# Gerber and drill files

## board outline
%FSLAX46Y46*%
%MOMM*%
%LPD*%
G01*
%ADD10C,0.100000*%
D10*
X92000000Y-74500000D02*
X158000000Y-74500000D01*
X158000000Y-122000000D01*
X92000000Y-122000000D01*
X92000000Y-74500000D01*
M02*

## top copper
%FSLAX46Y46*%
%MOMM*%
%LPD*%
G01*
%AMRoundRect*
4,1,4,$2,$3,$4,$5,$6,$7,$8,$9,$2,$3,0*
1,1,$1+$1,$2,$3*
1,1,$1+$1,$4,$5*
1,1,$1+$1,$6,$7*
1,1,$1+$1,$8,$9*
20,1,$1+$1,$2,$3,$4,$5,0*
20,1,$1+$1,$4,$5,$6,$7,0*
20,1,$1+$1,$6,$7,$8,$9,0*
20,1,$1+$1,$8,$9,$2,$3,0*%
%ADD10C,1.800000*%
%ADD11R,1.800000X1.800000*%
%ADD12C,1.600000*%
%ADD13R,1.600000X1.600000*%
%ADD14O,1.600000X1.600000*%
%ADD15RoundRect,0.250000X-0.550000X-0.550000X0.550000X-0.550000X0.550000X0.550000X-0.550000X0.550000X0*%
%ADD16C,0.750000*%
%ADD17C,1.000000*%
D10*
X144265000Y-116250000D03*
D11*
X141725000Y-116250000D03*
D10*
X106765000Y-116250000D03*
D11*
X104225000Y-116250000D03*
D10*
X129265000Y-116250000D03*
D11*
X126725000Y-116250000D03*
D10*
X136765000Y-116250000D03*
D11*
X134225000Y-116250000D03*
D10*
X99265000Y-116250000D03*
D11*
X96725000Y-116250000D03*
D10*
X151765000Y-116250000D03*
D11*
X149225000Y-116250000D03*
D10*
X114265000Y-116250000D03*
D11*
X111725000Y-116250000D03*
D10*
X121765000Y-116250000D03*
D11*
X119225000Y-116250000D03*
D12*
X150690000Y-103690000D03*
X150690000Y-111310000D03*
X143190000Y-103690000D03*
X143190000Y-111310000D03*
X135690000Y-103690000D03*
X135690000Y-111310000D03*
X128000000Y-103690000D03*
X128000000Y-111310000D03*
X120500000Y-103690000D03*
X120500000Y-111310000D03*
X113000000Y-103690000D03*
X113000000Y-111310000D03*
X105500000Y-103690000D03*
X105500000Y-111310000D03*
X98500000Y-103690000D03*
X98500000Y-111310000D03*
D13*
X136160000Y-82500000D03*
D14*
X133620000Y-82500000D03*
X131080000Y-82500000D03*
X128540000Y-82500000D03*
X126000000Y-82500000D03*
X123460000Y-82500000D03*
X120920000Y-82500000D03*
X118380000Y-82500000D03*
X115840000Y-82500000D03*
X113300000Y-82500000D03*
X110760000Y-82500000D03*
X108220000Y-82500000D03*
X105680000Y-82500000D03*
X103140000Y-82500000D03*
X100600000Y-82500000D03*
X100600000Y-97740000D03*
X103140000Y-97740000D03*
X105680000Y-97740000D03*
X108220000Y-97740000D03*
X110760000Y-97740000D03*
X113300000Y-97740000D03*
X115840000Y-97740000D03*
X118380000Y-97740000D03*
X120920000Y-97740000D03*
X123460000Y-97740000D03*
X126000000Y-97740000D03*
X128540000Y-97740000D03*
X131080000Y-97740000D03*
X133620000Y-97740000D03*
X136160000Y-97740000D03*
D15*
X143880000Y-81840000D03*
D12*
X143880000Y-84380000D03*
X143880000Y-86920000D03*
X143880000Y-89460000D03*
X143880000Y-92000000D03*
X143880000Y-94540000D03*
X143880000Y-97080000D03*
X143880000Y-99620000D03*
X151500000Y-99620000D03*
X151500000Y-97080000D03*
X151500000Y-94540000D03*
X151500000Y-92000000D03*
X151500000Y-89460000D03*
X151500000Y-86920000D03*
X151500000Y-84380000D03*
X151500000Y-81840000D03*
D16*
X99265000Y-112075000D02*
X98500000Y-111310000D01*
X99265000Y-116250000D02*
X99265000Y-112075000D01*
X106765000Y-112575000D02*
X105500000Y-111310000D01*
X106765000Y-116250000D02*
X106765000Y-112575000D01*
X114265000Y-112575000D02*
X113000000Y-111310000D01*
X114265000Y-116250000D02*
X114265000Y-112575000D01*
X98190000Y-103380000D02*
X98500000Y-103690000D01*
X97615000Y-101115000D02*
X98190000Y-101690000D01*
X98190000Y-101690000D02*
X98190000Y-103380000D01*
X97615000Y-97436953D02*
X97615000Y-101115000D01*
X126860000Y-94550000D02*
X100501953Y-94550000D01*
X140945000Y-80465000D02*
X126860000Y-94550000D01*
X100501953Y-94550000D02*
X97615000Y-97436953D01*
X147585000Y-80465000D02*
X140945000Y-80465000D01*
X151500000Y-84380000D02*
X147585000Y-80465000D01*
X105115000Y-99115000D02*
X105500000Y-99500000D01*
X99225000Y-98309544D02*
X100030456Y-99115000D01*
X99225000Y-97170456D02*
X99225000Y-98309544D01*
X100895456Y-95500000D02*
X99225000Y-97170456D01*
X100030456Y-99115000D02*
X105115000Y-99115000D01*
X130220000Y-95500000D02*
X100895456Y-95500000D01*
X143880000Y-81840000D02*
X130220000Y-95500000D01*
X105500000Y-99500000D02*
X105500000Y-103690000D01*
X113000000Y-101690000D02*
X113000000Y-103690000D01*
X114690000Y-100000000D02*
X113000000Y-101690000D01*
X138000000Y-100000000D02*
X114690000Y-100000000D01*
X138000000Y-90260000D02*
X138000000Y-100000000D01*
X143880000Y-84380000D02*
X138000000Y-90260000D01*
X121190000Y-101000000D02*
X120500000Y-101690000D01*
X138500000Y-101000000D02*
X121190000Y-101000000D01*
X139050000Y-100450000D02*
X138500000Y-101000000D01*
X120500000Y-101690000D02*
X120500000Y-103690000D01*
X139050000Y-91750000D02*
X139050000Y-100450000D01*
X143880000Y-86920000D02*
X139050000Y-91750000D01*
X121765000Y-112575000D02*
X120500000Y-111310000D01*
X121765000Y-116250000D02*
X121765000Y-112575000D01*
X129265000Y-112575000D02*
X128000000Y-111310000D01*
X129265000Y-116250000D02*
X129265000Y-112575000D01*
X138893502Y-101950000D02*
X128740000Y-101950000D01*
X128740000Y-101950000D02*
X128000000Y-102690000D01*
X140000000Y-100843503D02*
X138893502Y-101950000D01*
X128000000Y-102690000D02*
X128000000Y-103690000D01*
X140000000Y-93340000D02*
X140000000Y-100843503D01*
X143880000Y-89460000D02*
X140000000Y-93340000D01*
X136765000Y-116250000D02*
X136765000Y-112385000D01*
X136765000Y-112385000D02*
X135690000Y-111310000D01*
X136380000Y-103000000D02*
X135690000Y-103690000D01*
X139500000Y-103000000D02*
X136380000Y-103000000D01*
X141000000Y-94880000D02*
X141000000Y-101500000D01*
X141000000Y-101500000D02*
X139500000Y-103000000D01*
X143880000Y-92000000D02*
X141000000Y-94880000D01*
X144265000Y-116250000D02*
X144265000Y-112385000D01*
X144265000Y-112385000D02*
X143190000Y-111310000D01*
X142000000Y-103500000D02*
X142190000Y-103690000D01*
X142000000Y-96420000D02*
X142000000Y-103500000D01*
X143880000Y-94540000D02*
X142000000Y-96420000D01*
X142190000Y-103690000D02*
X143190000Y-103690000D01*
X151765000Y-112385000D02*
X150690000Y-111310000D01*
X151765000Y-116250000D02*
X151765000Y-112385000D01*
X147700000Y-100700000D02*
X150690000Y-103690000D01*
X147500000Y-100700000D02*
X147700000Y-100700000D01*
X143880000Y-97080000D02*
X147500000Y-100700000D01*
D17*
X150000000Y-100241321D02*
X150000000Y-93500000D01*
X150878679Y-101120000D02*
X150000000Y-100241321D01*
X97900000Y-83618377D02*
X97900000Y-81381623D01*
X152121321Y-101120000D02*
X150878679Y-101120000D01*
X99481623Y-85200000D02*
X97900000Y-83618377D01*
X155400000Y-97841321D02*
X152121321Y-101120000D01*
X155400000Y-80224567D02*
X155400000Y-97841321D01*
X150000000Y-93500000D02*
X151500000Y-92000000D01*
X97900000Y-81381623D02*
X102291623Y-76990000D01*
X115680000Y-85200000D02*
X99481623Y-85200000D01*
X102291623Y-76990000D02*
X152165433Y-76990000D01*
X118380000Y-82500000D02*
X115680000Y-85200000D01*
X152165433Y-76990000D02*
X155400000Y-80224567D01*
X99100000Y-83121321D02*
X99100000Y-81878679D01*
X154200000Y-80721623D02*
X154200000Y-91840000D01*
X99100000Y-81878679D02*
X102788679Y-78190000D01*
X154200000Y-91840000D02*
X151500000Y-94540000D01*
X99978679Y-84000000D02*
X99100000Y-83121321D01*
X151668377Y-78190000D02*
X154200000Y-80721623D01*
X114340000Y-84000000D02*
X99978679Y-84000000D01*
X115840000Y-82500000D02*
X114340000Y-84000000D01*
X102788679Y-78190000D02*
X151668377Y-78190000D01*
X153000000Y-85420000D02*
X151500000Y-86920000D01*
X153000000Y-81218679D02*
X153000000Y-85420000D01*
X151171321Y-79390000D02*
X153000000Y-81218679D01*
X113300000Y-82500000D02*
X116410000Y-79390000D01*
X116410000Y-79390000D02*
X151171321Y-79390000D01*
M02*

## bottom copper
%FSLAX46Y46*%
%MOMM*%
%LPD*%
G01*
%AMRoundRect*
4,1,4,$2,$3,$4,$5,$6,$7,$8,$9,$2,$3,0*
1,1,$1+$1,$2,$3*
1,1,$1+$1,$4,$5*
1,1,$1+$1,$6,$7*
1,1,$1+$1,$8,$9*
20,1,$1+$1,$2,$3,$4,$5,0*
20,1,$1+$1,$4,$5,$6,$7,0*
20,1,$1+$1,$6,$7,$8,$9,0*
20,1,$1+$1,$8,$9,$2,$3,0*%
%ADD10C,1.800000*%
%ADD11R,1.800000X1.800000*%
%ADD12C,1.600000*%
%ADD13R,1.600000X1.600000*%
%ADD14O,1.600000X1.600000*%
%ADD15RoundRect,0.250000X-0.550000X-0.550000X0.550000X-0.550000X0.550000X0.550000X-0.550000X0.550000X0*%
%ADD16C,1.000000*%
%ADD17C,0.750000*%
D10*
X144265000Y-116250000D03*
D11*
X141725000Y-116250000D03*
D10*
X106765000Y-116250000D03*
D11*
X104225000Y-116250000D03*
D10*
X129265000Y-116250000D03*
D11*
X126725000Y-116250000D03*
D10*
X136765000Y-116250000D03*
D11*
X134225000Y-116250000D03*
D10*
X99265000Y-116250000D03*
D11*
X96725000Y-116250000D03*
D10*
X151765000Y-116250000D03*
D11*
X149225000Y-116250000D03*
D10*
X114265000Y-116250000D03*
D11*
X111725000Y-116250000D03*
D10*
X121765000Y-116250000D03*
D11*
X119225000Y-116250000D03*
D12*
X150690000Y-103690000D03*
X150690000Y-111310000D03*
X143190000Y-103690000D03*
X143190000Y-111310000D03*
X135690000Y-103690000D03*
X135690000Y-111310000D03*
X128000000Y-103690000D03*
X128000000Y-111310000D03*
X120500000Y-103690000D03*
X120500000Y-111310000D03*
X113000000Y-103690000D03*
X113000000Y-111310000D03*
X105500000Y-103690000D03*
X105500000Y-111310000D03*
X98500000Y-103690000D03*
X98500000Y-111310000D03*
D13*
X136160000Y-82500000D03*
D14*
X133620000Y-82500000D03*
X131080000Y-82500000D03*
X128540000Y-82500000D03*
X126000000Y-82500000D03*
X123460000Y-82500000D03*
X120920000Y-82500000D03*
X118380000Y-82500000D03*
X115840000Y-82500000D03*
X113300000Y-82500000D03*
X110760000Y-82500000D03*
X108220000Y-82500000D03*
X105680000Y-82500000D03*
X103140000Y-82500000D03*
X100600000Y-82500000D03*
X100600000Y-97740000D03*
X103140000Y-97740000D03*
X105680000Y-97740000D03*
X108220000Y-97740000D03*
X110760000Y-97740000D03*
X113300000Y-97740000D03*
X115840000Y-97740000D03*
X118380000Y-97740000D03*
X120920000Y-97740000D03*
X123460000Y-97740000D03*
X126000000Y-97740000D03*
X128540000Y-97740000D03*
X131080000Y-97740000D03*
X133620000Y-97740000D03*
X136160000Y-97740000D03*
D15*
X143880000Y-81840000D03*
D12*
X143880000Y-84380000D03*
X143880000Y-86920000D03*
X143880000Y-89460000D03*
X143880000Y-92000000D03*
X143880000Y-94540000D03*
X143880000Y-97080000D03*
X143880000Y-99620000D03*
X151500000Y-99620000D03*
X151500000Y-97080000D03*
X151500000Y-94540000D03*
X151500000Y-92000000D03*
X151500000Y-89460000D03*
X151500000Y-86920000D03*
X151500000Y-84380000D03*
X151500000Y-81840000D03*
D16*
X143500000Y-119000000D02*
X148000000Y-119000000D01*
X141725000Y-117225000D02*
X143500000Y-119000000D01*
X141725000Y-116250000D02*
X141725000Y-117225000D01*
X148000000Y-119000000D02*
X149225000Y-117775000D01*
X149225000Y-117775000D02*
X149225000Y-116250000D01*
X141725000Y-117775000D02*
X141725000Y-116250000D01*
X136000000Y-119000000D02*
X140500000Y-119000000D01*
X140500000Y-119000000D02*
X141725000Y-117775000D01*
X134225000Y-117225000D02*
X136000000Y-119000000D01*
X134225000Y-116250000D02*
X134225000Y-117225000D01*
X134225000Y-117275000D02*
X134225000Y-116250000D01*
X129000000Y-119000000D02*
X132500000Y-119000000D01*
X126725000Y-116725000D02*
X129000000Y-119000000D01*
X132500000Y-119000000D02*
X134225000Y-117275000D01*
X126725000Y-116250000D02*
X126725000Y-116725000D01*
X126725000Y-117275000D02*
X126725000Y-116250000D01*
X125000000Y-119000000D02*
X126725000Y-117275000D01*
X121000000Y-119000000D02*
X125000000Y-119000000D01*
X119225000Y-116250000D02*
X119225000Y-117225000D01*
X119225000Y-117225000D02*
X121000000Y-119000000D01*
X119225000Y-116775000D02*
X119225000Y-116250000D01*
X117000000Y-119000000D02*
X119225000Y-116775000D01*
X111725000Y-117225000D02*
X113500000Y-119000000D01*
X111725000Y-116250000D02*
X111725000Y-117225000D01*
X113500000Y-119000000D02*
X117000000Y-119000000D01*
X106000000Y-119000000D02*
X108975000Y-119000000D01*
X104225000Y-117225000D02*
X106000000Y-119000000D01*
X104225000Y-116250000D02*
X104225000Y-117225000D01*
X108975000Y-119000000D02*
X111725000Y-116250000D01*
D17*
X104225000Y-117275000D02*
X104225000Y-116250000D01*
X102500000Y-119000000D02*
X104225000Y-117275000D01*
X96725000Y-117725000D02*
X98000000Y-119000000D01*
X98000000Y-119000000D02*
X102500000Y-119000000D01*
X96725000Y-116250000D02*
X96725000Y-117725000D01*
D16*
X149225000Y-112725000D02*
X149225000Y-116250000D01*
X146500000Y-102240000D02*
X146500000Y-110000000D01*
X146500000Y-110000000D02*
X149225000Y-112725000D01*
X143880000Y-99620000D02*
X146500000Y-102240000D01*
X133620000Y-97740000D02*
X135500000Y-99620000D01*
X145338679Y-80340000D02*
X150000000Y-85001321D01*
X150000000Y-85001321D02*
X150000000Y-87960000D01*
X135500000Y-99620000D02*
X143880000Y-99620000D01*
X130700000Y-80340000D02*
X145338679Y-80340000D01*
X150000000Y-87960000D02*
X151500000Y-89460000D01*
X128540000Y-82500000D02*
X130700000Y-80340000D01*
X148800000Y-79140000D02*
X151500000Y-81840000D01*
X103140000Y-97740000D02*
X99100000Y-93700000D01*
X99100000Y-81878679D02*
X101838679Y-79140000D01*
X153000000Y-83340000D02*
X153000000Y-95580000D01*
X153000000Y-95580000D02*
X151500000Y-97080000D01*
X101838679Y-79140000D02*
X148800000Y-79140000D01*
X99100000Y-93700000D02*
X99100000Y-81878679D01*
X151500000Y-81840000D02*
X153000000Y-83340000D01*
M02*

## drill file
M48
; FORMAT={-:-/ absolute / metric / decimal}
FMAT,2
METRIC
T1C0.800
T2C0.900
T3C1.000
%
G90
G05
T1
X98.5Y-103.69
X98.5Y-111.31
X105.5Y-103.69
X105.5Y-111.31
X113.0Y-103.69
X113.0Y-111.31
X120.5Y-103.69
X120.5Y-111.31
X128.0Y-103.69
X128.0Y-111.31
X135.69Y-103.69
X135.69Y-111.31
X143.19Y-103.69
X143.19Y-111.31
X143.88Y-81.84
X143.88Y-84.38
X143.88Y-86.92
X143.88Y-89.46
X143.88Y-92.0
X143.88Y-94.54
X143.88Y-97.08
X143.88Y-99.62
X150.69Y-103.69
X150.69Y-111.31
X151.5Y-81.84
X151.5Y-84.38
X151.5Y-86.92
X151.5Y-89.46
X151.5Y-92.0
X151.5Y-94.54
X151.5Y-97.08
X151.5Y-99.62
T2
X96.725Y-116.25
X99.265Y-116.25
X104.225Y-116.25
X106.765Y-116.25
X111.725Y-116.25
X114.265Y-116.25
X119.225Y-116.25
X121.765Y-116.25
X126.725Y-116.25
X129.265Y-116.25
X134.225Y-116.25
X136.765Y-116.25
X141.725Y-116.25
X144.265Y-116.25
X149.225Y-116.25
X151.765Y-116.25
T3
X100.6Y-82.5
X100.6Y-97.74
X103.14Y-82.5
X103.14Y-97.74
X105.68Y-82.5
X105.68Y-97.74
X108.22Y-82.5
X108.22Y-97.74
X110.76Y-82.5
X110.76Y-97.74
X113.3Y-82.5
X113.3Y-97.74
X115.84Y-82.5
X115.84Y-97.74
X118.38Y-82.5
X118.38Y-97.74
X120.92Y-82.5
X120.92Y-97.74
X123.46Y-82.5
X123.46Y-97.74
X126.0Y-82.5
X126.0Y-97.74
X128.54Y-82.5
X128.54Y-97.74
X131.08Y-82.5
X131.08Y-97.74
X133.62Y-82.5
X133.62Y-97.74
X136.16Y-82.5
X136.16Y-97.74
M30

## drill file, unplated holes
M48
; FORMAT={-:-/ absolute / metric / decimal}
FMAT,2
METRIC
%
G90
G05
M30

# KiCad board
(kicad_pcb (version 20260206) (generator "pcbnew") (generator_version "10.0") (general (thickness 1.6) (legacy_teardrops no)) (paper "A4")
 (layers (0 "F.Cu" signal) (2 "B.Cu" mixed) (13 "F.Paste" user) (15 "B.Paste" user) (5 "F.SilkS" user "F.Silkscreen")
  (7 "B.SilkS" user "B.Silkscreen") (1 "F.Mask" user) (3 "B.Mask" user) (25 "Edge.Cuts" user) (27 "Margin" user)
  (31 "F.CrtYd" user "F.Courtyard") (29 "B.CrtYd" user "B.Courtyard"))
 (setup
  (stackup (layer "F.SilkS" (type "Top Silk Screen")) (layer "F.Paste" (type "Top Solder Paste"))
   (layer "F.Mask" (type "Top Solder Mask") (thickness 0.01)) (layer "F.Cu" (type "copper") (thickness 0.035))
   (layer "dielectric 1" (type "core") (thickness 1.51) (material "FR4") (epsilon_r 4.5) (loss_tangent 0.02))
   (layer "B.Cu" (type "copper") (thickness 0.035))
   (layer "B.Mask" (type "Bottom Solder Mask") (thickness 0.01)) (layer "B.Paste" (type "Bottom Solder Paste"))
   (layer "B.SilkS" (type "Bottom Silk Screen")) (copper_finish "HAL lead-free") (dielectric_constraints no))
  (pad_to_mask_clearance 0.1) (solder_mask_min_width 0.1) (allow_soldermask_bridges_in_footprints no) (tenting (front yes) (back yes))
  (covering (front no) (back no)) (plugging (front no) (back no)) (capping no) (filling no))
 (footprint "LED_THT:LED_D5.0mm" (layer "F.Cu") (at 119.225 116.25)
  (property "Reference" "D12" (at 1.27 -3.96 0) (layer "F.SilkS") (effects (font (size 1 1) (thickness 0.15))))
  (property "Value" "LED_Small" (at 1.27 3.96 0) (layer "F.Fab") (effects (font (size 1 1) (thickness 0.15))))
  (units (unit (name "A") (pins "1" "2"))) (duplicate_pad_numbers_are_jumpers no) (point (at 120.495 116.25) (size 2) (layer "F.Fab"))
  (pad "1" thru_hole rect (at 0 0) (size 1.8 1.8) (drill 0.9) (layers "*.Cu" "*.Mask") (remove_unused_layers no) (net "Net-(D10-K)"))
  (pad "2" thru_hole circle (at 2.54 0) (size 1.8 1.8) (drill 0.9) (layers "*.Cu" "*.Mask") (remove_unused_layers no) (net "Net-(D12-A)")))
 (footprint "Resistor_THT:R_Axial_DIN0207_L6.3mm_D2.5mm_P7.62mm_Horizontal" (layer "F.Cu") (at 128 103.69 -90)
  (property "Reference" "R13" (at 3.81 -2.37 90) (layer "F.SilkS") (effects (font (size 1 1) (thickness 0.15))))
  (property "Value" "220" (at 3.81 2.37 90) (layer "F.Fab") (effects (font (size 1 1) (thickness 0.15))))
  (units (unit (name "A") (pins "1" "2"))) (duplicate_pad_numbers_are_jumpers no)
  (pad "1" thru_hole circle (at 0 0 270) (size 1.6 1.6) (drill 0.8) (layers "*.Cu" "*.Mask") (remove_unused_layers no) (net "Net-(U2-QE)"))
  (pad "2" thru_hole circle (at 7.62 0 270) (size 1.6 1.6) (drill 0.8) (layers "*.Cu" "*.Mask") (remove_unused_layers no)
   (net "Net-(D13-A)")))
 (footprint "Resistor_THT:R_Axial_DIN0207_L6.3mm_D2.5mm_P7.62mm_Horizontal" (layer "F.Cu") (at 150.69 103.69 -90)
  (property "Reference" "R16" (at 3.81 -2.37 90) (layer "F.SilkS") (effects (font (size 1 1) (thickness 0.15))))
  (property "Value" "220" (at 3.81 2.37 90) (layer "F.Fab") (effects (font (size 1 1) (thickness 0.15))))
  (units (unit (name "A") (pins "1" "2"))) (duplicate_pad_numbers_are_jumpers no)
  (pad "1" thru_hole circle (at 0 0 270) (size 1.6 1.6) (drill 0.8) (layers "*.Cu" "*.Mask") (remove_unused_layers no) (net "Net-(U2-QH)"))
  (pad "2" thru_hole circle (at 7.62 0 270) (size 1.6 1.6) (drill 0.8) (layers "*.Cu" "*.Mask") (remove_unused_layers no)
   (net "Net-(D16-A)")))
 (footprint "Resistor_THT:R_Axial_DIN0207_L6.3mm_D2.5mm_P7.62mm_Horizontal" (layer "F.Cu") (at 135.69 103.69 -90)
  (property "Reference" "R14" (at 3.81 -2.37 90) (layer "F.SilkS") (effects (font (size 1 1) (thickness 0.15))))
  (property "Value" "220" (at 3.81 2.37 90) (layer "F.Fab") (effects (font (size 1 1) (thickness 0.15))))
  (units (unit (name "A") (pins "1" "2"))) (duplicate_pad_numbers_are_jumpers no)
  (pad "1" thru_hole circle (at 0 0 270) (size 1.6 1.6) (drill 0.8) (layers "*.Cu" "*.Mask") (remove_unused_layers no) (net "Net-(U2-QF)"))
  (pad "2" thru_hole circle (at 7.62 0 270) (size 1.6 1.6) (drill 0.8) (layers "*.Cu" "*.Mask") (remove_unused_layers no)
   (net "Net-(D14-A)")))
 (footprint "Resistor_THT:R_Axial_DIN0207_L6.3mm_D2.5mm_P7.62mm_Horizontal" (layer "F.Cu") (at 113 103.69 -90)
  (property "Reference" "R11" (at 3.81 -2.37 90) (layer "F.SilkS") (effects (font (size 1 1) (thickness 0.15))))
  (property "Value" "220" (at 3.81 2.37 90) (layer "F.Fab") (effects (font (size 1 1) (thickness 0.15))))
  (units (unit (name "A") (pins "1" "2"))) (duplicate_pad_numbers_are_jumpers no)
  (pad "1" thru_hole circle (at 0 0 270) (size 1.6 1.6) (drill 0.8) (layers "*.Cu" "*.Mask") (remove_unused_layers no) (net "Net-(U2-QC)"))
  (pad "2" thru_hole circle (at 7.62 0 270) (size 1.6 1.6) (drill 0.8) (layers "*.Cu" "*.Mask") (remove_unused_layers no)
   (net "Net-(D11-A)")))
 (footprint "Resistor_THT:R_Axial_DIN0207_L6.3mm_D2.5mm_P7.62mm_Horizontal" (layer "F.Cu") (at 105.5 103.69 -90)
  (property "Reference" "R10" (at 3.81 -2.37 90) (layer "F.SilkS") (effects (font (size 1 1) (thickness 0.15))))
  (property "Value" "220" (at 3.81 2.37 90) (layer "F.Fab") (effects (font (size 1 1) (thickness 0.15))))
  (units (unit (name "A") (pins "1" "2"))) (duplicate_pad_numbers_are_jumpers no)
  (pad "1" thru_hole circle (at 0 0 270) (size 1.6 1.6) (drill 0.8) (layers "*.Cu" "*.Mask") (remove_unused_layers no) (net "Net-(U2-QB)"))
  (pad "2" thru_hole circle (at 7.62 0 270) (size 1.6 1.6) (drill 0.8) (layers "*.Cu" "*.Mask") (remove_unused_layers no)
   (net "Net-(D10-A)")))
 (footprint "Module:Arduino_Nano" (layer "F.Cu") (at 136.16 82.5 -90)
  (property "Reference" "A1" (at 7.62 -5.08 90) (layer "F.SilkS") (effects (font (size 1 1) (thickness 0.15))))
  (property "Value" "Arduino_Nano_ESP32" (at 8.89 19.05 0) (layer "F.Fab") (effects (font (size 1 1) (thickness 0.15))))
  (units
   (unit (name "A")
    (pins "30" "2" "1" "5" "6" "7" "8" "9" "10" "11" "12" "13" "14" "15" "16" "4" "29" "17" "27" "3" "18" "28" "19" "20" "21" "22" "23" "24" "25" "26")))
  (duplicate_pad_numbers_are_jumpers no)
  (pad "1" thru_hole rect (at 0 0 270) (size 1.6 1.6) (drill 1) (layers "*.Cu" "*.Mask") (remove_unused_layers no)
   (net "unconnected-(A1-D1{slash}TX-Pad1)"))
  (pad "2" thru_hole oval (at 0 2.54 270) (size 1.6 1.6) (drill 1) (layers "*.Cu" "*.Mask") (remove_unused_layers no)
   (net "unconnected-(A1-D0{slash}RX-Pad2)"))
  (pad "3" thru_hole oval (at 0 5.08 270) (size 1.6 1.6) (drill 1) (layers "*.Cu" "*.Mask") (remove_unused_layers no)
   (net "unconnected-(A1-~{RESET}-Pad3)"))
  (pad "4" thru_hole oval (at 0 7.62 270) (size 1.6 1.6) (drill 1) (layers "*.Cu" "*.Mask") (remove_unused_layers no) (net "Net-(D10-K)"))
  (pad "5" thru_hole oval (at 0 10.16 270) (size 1.6 1.6) (drill 1) (layers "*.Cu" "*.Mask") (remove_unused_layers no)
   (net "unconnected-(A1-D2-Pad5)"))
  (pad "6" thru_hole oval (at 0 12.7 270) (size 1.6 1.6) (drill 1) (layers "*.Cu" "*.Mask") (remove_unused_layers no)
   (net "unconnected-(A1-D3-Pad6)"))
  (pad "7" thru_hole oval (at 0 15.24 270) (size 1.6 1.6) (drill 1) (layers "*.Cu" "*.Mask") (remove_unused_layers no)
   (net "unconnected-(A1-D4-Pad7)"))
  (pad "8" thru_hole oval (at 0 17.78 270) (size 1.6 1.6) (drill 1) (layers "*.Cu" "*.Mask") (remove_unused_layers no) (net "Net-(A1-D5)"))
  (pad "9" thru_hole oval (at 0 20.32 270) (size 1.6 1.6) (drill 1) (layers "*.Cu" "*.Mask") (remove_unused_layers no) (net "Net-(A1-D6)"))
  (pad "10" thru_hole oval (at 0 22.86 270) (size 1.6 1.6) (drill 1) (layers "*.Cu" "*.Mask") (remove_unused_layers no) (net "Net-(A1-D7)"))
  (pad "11" thru_hole oval (at 0 25.4 270) (size 1.6 1.6) (drill 1) (layers "*.Cu" "*.Mask") (remove_unused_layers no)
   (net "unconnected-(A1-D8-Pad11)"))
  (pad "12" thru_hole oval (at 0 27.94 270) (size 1.6 1.6) (drill 1) (layers "*.Cu" "*.Mask") (remove_unused_layers no)
   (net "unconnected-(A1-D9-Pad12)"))
  (pad "13" thru_hole oval (at 0 30.48 270) (size 1.6 1.6) (drill 1) (layers "*.Cu" "*.Mask") (remove_unused_layers no)
   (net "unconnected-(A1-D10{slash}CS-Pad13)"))
  (pad "14" thru_hole oval (at 0 33.02 270) (size 1.6 1.6) (drill 1) (layers "*.Cu" "*.Mask") (remove_unused_layers no)
   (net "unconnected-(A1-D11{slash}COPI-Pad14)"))
  (pad "15" thru_hole oval (at 0 35.56 270) (size 1.6 1.6) (drill 1) (layers "*.Cu" "*.Mask") (remove_unused_layers no)
   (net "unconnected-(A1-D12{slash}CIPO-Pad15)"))
  (pad "16" thru_hole oval (at 15.24 35.56 270) (size 1.6 1.6) (drill 1) (layers "*.Cu" "*.Mask") (remove_unused_layers no)
   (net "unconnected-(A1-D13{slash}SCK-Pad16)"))
  (pad "17" thru_hole oval (at 15.24 33.02 270) (size 1.6 1.6) (drill 1) (layers "*.Cu" "*.Mask") (remove_unused_layers no)
   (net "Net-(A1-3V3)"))
  (pad "18" thru_hole oval (at 15.24 30.48 270) (size 1.6 1.6) (drill 1) (layers "*.Cu" "*.Mask") (remove_unused_layers no)
   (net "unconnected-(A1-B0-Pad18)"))
  (pad "19" thru_hole oval (at 15.24 27.94 270) (size 1.6 1.6) (drill 1) (layers "*.Cu" "*.Mask") (remove_unused_layers no)
   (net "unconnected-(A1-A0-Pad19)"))
  (pad "20" thru_hole oval (at 15.24 25.4 270) (size 1.6 1.6) (drill 1) (layers "*.Cu" "*.Mask") (remove_unused_layers no)
   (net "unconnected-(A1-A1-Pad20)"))
  (pad "21" thru_hole oval (at 15.24 22.86 270) (size 1.6 1.6) (drill 1) (layers "*.Cu" "*.Mask") (remove_unused_layers no)
   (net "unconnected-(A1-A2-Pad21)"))
  (pad "22" thru_hole oval (at 15.24 20.32 270) (size 1.6 1.6) (drill 1) (layers "*.Cu" "*.Mask") (remove_unused_layers no)
   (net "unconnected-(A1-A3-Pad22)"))
  (pad "23" thru_hole oval (at 15.24 17.78 270) (size 1.6 1.6) (drill 1) (layers "*.Cu" "*.Mask") (remove_unused_layers no)
   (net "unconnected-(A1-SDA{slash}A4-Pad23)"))
  (pad "24" thru_hole oval (at 15.24 15.24 270) (size 1.6 1.6) (drill 1) (layers "*.Cu" "*.Mask") (remove_unused_layers no)
   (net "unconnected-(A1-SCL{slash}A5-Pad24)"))
  (pad "25" thru_hole oval (at 15.24 12.7 270) (size 1.6 1.6) (drill 1) (layers "*.Cu" "*.Mask") (remove_unused_layers no)
   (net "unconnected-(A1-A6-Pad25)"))
  (pad "26" thru_hole oval (at 15.24 10.16 270) (size 1.6 1.6) (drill 1) (layers "*.Cu" "*.Mask") (remove_unused_layers no)
   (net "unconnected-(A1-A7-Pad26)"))
  (pad "27" thru_hole oval (at 15.24 7.62 270) (size 1.6 1.6) (drill 1) (layers "*.Cu" "*.Mask") (remove_unused_layers no)
   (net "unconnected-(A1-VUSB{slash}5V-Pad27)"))
  (pad "28" thru_hole oval (at 15.24 5.08 270) (size 1.6 1.6) (drill 1) (layers "*.Cu" "*.Mask") (remove_unused_layers no)
   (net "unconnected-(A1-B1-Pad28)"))
  (pad "29" thru_hole oval (at 15.24 2.54 270) (size 1.6 1.6) (drill 1) (layers "*.Cu" "*.Mask") (remove_unused_layers no)
   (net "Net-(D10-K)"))
  (pad "30" thru_hole oval (at 15.24 0 270) (size 1.6 1.6) (drill 1) (layers "*.Cu" "*.Mask") (remove_unused_layers no)
   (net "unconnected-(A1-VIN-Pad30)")))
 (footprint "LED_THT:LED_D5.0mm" (layer "F.Cu") (at 104.225 116.25)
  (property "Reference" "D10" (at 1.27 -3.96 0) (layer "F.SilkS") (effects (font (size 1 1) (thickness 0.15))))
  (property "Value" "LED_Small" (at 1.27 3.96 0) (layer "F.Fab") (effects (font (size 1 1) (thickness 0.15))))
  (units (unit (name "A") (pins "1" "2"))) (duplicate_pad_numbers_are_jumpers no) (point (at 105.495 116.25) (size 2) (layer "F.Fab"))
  (pad "1" thru_hole rect (at 0 0) (size 1.8 1.8) (drill 0.9) (layers "*.Cu" "*.Mask") (remove_unused_layers no) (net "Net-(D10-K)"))
  (pad "2" thru_hole circle (at 2.54 0) (size 1.8 1.8) (drill 0.9) (layers "*.Cu" "*.Mask") (remove_unused_layers no) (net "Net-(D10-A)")))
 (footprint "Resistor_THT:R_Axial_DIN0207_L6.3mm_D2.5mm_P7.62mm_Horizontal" (layer "F.Cu") (at 143.19 103.69 -90)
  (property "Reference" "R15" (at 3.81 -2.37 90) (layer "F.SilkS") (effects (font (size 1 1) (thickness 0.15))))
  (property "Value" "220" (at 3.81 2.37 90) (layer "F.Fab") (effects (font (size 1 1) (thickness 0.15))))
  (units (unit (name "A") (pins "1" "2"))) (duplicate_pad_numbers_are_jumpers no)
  (pad "1" thru_hole circle (at 0 0 270) (size 1.6 1.6) (drill 0.8) (layers "*.Cu" "*.Mask") (remove_unused_layers no) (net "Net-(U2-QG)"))
  (pad "2" thru_hole circle (at 7.62 0 270) (size 1.6 1.6) (drill 0.8) (layers "*.Cu" "*.Mask") (remove_unused_layers no)
   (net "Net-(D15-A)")))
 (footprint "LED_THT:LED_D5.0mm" (layer "F.Cu") (at 126.725 116.25)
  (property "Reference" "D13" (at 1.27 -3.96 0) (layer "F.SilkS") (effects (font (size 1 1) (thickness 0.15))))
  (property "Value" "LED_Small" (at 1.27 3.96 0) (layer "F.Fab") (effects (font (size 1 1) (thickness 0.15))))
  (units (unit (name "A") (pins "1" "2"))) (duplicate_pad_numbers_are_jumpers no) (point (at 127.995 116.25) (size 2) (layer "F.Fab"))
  (pad "1" thru_hole rect (at 0 0) (size 1.8 1.8) (drill 0.9) (layers "*.Cu" "*.Mask") (remove_unused_layers no) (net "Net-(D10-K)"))
  (pad "2" thru_hole circle (at 2.54 0) (size 1.8 1.8) (drill 0.9) (layers "*.Cu" "*.Mask") (remove_unused_layers no) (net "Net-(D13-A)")))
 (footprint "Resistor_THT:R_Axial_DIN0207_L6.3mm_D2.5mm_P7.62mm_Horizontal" (layer "F.Cu") (at 120.5 103.69 -90)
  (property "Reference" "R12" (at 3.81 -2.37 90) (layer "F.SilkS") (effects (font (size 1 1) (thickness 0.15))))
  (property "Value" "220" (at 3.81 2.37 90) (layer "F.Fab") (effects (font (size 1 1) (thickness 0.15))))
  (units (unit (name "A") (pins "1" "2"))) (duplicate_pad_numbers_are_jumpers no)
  (pad "1" thru_hole circle (at 0 0 270) (size 1.6 1.6) (drill 0.8) (layers "*.Cu" "*.Mask") (remove_unused_layers no) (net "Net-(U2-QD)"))
  (pad "2" thru_hole circle (at 7.62 0 270) (size 1.6 1.6) (drill 0.8) (layers "*.Cu" "*.Mask") (remove_unused_layers no)
   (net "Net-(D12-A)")))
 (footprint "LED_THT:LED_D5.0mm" (layer "F.Cu") (at 141.725 116.25)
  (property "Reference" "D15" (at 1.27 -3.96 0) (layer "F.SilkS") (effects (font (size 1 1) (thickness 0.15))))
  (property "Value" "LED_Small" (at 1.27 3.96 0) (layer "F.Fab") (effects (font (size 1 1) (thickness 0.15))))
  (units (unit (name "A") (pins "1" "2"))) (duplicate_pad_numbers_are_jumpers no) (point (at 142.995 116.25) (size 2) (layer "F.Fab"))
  (pad "1" thru_hole rect (at 0 0) (size 1.8 1.8) (drill 0.9) (layers "*.Cu" "*.Mask") (remove_unused_layers no) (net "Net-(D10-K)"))
  (pad "2" thru_hole circle (at 2.54 0) (size 1.8 1.8) (drill 0.9) (layers "*.Cu" "*.Mask") (remove_unused_layers no) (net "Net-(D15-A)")))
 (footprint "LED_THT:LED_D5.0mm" (layer "F.Cu") (at 111.725 116.25)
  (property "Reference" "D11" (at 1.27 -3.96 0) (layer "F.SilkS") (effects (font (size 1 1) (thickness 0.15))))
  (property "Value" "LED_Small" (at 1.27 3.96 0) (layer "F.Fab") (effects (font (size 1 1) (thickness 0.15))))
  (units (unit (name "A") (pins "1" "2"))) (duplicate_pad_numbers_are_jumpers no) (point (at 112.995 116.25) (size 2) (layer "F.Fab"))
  (pad "1" thru_hole rect (at 0 0) (size 1.8 1.8) (drill 0.9) (layers "*.Cu" "*.Mask") (remove_unused_layers no) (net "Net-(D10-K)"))
  (pad "2" thru_hole circle (at 2.54 0) (size 1.8 1.8) (drill 0.9) (layers "*.Cu" "*.Mask") (remove_unused_layers no) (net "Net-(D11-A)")))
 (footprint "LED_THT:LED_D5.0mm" (layer "F.Cu") (at 149.225 116.25)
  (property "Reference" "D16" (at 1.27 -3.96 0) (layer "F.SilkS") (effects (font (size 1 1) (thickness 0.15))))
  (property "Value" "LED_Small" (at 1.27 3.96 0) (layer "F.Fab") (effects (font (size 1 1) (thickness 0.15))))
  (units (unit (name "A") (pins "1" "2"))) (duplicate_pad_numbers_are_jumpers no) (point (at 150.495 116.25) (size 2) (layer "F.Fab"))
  (pad "1" thru_hole rect (at 0 0) (size 1.8 1.8) (drill 0.9) (layers "*.Cu" "*.Mask") (remove_unused_layers no) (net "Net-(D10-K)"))
  (pad "2" thru_hole circle (at 2.54 0) (size 1.8 1.8) (drill 0.9) (layers "*.Cu" "*.Mask") (remove_unused_layers no) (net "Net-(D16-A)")))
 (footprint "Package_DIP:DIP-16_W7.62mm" (layer "F.Cu") (at 143.88 81.84)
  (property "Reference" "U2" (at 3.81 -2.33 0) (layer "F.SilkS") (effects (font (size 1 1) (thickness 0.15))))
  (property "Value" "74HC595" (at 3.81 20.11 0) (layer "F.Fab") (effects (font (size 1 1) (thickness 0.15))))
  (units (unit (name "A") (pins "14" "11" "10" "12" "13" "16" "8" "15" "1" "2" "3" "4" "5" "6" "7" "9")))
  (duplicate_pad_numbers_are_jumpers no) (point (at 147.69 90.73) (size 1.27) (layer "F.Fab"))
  (pad "1" thru_hole roundrect (at 0 0) (size 1.6 1.6) (drill 0.8) (layers "*.Cu" "*.Mask") (remove_unused_layers no)
   (roundrect_rratio 0.15625) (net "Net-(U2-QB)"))
  (pad "2" thru_hole circle (at 0 2.54) (size 1.6 1.6) (drill 0.8) (layers "*.Cu" "*.Mask") (remove_unused_layers no) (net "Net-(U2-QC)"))
  (pad "3" thru_hole circle (at 0 5.08) (size 1.6 1.6) (drill 0.8) (layers "*.Cu" "*.Mask") (remove_unused_layers no) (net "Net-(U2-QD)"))
  (pad "4" thru_hole circle (at 0 7.62) (size 1.6 1.6) (drill 0.8) (layers "*.Cu" "*.Mask") (remove_unused_layers no) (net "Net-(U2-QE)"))
  (pad "5" thru_hole circle (at 0 10.16) (size 1.6 1.6) (drill 0.8) (layers "*.Cu" "*.Mask") (remove_unused_layers no) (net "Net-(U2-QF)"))
  (pad "6" thru_hole circle (at 0 12.7) (size 1.6 1.6) (drill 0.8) (layers "*.Cu" "*.Mask") (remove_unused_layers no) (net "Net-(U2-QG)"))
  (pad "7" thru_hole circle (at 0 15.24) (size 1.6 1.6) (drill 0.8) (layers "*.Cu" "*.Mask") (remove_unused_layers no) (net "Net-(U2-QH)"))
  (pad "8" thru_hole circle (at 0 17.78) (size 1.6 1.6) (drill 0.8) (layers "*.Cu" "*.Mask") (remove_unused_layers no) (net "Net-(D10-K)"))
  (pad "9" thru_hole circle (at 7.62 17.78) (size 1.6 1.6) (drill 0.8) (layers "*.Cu" "*.Mask") (remove_unused_layers no)
   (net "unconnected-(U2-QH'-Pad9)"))
  (pad "10" thru_hole circle (at 7.62 15.24) (size 1.6 1.6) (drill 0.8) (layers "*.Cu" "*.Mask") (remove_unused_layers no)
   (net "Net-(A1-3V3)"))
  (pad "11" thru_hole circle (at 7.62 12.7) (size 1.6 1.6) (drill 0.8) (layers "*.Cu" "*.Mask") (remove_unused_layers no)
   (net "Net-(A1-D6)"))
  (pad "12" thru_hole circle (at 7.62 10.16) (size 1.6 1.6) (drill 0.8) (layers "*.Cu" "*.Mask") (remove_unused_layers no)
   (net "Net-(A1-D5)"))
  (pad "13" thru_hole circle (at 7.62 7.62) (size 1.6 1.6) (drill 0.8) (layers "*.Cu" "*.Mask") (remove_unused_layers no)
   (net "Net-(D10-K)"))
  (pad "14" thru_hole circle (at 7.62 5.08) (size 1.6 1.6) (drill 0.8) (layers "*.Cu" "*.Mask") (remove_unused_layers no)
   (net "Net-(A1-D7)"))
  (pad "15" thru_hole circle (at 7.62 2.54) (size 1.6 1.6) (drill 0.8) (layers "*.Cu" "*.Mask") (remove_unused_layers no)
   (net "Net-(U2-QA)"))
  (pad "16" thru_hole circle (at 7.62 0) (size 1.6 1.6) (drill 0.8) (layers "*.Cu" "*.Mask") (remove_unused_layers no) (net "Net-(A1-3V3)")))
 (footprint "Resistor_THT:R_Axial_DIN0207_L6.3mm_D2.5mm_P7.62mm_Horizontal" (layer "F.Cu") (at 98.5 103.69 -90)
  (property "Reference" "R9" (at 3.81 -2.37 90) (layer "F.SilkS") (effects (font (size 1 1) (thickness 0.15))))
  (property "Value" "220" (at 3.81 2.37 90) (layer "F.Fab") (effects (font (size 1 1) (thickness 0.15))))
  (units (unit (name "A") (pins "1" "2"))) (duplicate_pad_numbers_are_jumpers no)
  (pad "1" thru_hole circle (at 0 0 270) (size 1.6 1.6) (drill 0.8) (layers "*.Cu" "*.Mask") (remove_unused_layers no) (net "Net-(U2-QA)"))
  (pad "2" thru_hole circle (at 7.62 0 270) (size 1.6 1.6) (drill 0.8) (layers "*.Cu" "*.Mask") (remove_unused_layers no) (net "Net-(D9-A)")))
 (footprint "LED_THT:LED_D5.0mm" (layer "F.Cu") (at 96.725 116.25)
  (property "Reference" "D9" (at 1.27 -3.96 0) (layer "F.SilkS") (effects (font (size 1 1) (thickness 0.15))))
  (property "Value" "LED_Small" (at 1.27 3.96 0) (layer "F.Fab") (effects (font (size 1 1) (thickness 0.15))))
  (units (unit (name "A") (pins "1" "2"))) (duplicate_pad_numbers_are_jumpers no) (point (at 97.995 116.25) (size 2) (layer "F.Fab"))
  (pad "1" thru_hole rect (at 0 0) (size 1.8 1.8) (drill 0.9) (layers "*.Cu" "*.Mask") (remove_unused_layers no) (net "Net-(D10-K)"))
  (pad "2" thru_hole circle (at 2.54 0) (size 1.8 1.8) (drill 0.9) (layers "*.Cu" "*.Mask") (remove_unused_layers no) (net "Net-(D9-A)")))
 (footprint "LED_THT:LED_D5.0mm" (layer "F.Cu") (at 134.225 116.25)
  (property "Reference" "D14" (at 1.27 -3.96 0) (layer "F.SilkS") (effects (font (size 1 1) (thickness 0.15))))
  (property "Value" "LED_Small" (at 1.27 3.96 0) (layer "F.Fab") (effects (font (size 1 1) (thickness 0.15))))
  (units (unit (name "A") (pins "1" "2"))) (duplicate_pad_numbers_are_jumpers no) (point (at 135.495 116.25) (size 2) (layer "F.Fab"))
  (pad "1" thru_hole rect (at 0 0) (size 1.8 1.8) (drill 0.9) (layers "*.Cu" "*.Mask") (remove_unused_layers no) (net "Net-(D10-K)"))
  (pad "2" thru_hole circle (at 2.54 0) (size 1.8 1.8) (drill 0.9) (layers "*.Cu" "*.Mask") (remove_unused_layers no) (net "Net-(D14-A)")))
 (gr_rect (start 92 74.5) (end 158 122) (stroke (width 0.1) (type default)) (fill no) (layer "Edge.Cuts"))
 (segment (start 134.225 116.25) (end 134.225 117.225) (width 1) (layer "B.Cu") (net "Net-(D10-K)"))
 (segment (start 98 119) (end 102.5 119) (width 0.75) (layer "B.Cu") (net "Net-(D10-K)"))
 (segment (start 143.5 119) (end 148 119) (width 1) (layer "B.Cu") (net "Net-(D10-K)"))
 (segment (start 146.5 110) (end 149.225 112.725) (width 1) (layer "B.Cu") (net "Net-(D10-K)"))
 (segment (start 126.725 116.25) (end 126.725 116.725) (width 1) (layer "B.Cu") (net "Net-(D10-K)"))
 (segment (start 96.725 117.725) (end 98 119) (width 0.75) (layer "B.Cu") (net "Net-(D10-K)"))
 (segment (start 102.5 119) (end 104.225 117.275) (width 0.75) (layer "B.Cu") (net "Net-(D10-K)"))
 (segment (start 134.225 117.225) (end 136 119) (width 1) (layer "B.Cu") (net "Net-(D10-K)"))
 (segment (start 143.88 99.62) (end 146.5 102.24) (width 1) (layer "B.Cu") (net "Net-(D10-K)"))
 (segment (start 133.62 97.74) (end 135.5 99.62) (width 1) (layer "B.Cu") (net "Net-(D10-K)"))
 (segment (start 136 119) (end 140.5 119) (width 1) (layer "B.Cu") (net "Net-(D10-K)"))
 (segment (start 149.225 117.775) (end 149.225 116.25) (width 1) (layer "B.Cu") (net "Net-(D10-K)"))
 (segment (start 125 119) (end 126.725 117.275) (width 1) (layer "B.Cu") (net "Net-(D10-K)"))
 (segment (start 113.5 119) (end 117 119) (width 1) (layer "B.Cu") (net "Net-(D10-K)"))
 (segment (start 141.725 117.775) (end 141.725 116.25) (width 1) (layer "B.Cu") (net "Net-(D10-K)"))
 (segment (start 145.338679 80.34) (end 150 85.001321) (width 1) (layer "B.Cu") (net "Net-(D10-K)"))
 (segment (start 129 119) (end 132.5 119) (width 1) (layer "B.Cu") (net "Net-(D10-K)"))
 (segment (start 126.725 116.725) (end 129 119) (width 1) (layer "B.Cu") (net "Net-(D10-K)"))
 (segment (start 108.975 119) (end 111.725 116.25) (width 1) (layer "B.Cu") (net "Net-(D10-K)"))
 (segment (start 150 85.001321) (end 150 87.96) (width 1) (layer "B.Cu") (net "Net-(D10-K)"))
 (segment (start 134.225 117.275) (end 134.225 116.25) (width 1) (layer "B.Cu") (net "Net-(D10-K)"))
 (segment (start 126.725 117.275) (end 126.725 116.25) (width 1) (layer "B.Cu") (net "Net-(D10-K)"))
 (segment (start 135.5 99.62) (end 143.88 99.62) (width 1) (layer "B.Cu") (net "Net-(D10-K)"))
 (segment (start 111.725 117.225) (end 113.5 119) (width 1) (layer "B.Cu") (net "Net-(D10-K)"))
 (segment (start 140.5 119) (end 141.725 117.775) (width 1) (layer "B.Cu") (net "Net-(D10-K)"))
 (segment (start 104.225 117.225) (end 106 119) (width 1) (layer "B.Cu") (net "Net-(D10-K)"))
 (segment (start 119.225 116.775) (end 119.225 116.25) (width 1) (layer "B.Cu") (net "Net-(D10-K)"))
 (segment (start 148 119) (end 149.225 117.775) (width 1) (layer "B.Cu") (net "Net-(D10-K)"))
 (segment (start 130.7 80.34) (end 145.338679 80.34) (width 1) (layer "B.Cu") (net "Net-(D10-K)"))
 (segment (start 121 119) (end 125 119) (width 1) (layer "B.Cu") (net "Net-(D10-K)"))
 (segment (start 104.225 116.25) (end 104.225 117.225) (width 1) (layer "B.Cu") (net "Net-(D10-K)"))
 (segment (start 106 119) (end 108.975 119) (width 1) (layer "B.Cu") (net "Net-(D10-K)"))
 (segment (start 119.225 116.25) (end 119.225 117.225) (width 1) (layer "B.Cu") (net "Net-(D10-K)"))
 (segment (start 104.225 117.275) (end 104.225 116.25) (width 0.75) (layer "B.Cu") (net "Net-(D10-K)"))
 (segment (start 141.725 116.25) (end 141.725 117.225) (width 1) (layer "B.Cu") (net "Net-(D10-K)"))
 (segment (start 119.225 117.225) (end 121 119) (width 1) (layer "B.Cu") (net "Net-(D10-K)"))
 (segment (start 150 87.96) (end 151.5 89.46) (width 1) (layer "B.Cu") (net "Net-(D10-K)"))
 (segment (start 111.725 116.25) (end 111.725 117.225) (width 1) (layer "B.Cu") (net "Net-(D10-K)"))
 (segment (start 128.54 82.5) (end 130.7 80.34) (width 1) (layer "B.Cu") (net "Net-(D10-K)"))
 (segment (start 141.725 117.225) (end 143.5 119) (width 1) (layer "B.Cu") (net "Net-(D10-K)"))
 (segment (start 149.225 112.725) (end 149.225 116.25) (width 1) (layer "B.Cu") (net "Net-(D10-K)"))
 (segment (start 117 119) (end 119.225 116.775) (width 1) (layer "B.Cu") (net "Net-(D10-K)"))
 (segment (start 146.5 102.24) (end 146.5 110) (width 1) (layer "B.Cu") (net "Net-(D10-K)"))
 (segment (start 132.5 119) (end 134.225 117.275) (width 1) (layer "B.Cu") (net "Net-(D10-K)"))
 (segment (start 96.725 116.25) (end 96.725 117.725) (width 0.75) (layer "B.Cu") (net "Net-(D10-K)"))
 (segment (start 121.765 112.575) (end 120.5 111.31) (width 0.75) (layer "F.Cu") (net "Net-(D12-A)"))
 (segment (start 121.765 116.25) (end 121.765 112.575) (width 0.75) (layer "F.Cu") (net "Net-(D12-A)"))
 (segment (start 143.88 89.46) (end 140 93.34) (width 0.75) (layer "F.Cu") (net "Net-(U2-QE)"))
 (segment (start 128 102.69) (end 128 103.69) (width 0.75) (layer "F.Cu") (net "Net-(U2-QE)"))
 (segment (start 128.74 101.95) (end 128 102.69) (width 0.75) (layer "F.Cu") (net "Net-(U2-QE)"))
 (segment (start 138.893502 101.95) (end 128.74 101.95) (width 0.75) (layer "F.Cu") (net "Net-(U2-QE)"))
 (segment (start 140 100.843503) (end 138.893502 101.95) (width 0.75) (layer "F.Cu") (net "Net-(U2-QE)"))
 (segment (start 140 93.34) (end 140 100.843503) (width 0.75) (layer "F.Cu") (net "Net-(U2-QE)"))
 (segment (start 129.265 112.575) (end 128 111.31) (width 0.75) (layer "F.Cu") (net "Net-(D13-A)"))
 (segment (start 129.265 116.25) (end 129.265 112.575) (width 0.75) (layer "F.Cu") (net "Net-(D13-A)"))
 (segment (start 147.5 100.7) (end 147.7 100.7) (width 0.75) (layer "F.Cu") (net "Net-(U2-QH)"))
 (segment (start 147.7 100.7) (end 150.69 103.69) (width 0.75) (layer "F.Cu") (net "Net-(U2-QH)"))
 (segment (start 143.88 97.08) (end 147.5 100.7) (width 0.75) (layer "F.Cu") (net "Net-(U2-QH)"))
 (segment (start 151.765 112.385) (end 150.69 111.31) (width 0.75) (layer "F.Cu") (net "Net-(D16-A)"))
 (segment (start 151.765 116.25) (end 151.765 112.385) (width 0.75) (layer "F.Cu") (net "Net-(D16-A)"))
 (segment (start 141 94.88) (end 141 101.5) (width 0.75) (layer "F.Cu") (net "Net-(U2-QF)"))
 (segment (start 141 101.5) (end 139.5 103) (width 0.75) (layer "F.Cu") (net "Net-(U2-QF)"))
 (segment (start 139.5 103) (end 136.38 103) (width 0.75) (layer "F.Cu") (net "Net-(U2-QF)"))
 (segment (start 136.38 103) (end 135.69 103.69) (width 0.75) (layer "F.Cu") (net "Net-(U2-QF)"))
 (segment (start 143.88 92) (end 141 94.88) (width 0.75) (layer "F.Cu") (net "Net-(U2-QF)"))
 (segment (start 136.765 116.25) (end 136.765 112.385) (width 0.75) (layer "F.Cu") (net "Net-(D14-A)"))
 (segment (start 136.765 112.385) (end 135.69 111.31) (width 0.75) (layer "F.Cu") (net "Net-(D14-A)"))
 (segment (start 143.88 84.38) (end 138 90.26) (width 0.75) (layer "F.Cu") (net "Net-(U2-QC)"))
 (segment (start 114.69 100) (end 113 101.69) (width 0.75) (layer "F.Cu") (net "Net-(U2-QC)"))
 (segment (start 113 101.69) (end 113 103.69) (width 0.75) (layer "F.Cu") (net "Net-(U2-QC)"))
 (segment (start 138 100) (end 114.69 100) (width 0.75) (layer "F.Cu") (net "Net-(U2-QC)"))
 (segment (start 138 90.26) (end 138 100) (width 0.75) (layer "F.Cu") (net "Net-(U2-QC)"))
 (segment (start 114.265 112.575) (end 113 111.31) (width 0.75) (layer "F.Cu") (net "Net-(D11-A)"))
 (segment (start 114.265 116.25) (end 114.265 112.575) (width 0.75) (layer "F.Cu") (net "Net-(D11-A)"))
 (segment (start 99.225 97.170456) (end 99.225 98.309544) (width 0.75) (layer "F.Cu") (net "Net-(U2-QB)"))
 (segment (start 130.22 95.5) (end 100.895456 95.5) (width 0.75) (layer "F.Cu") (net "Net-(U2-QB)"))
 (segment (start 105.5 99.5) (end 105.5 103.69) (width 0.75) (layer "F.Cu") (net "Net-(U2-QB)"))
 (segment (start 100.030456 99.115) (end 105.115 99.115) (width 0.75) (layer "F.Cu") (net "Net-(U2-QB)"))
 (segment (start 99.225 98.309544) (end 100.030456 99.115) (width 0.75) (layer "F.Cu") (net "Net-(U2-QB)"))
 (segment (start 105.115 99.115) (end 105.5 99.5) (width 0.75) (layer "F.Cu") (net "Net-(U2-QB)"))
 (segment (start 100.895456 95.5) (end 99.225 97.170456) (width 0.75) (layer "F.Cu") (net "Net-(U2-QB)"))
 (segment (start 143.88 81.84) (end 130.22 95.5) (width 0.75) (layer "F.Cu") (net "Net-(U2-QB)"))
 (segment (start 106.765 112.575) (end 105.5 111.31) (width 0.75) (layer "F.Cu") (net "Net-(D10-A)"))
 (segment (start 106.765 116.25) (end 106.765 112.575) (width 0.75) (layer "F.Cu") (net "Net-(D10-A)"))
 (segment (start 150 100.241321) (end 150 93.5) (width 1) (layer "F.Cu") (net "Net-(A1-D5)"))
 (segment (start 150.878679 101.12) (end 150 100.241321) (width 1) (layer "F.Cu") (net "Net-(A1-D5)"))
 (segment (start 97.9 83.618377) (end 97.9 81.381623) (width 1) (layer "F.Cu") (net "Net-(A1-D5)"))
 (segment (start 152.121321 101.12) (end 150.878679 101.12) (width 1) (layer "F.Cu") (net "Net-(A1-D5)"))
 (segment (start 99.481623 85.2) (end 97.9 83.618377) (width 1) (layer "F.Cu") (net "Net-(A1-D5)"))
 (segment (start 155.4 97.841321) (end 152.121321 101.12) (width 1) (layer "F.Cu") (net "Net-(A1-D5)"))
 (segment (start 155.4 80.224567) (end 155.4 97.841321) (width 1) (layer "F.Cu") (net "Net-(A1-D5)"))
 (segment (start 150 93.5) (end 151.5 92) (width 1) (layer "F.Cu") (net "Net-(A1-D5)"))
 (segment (start 97.9 81.381623) (end 102.291623 76.99) (width 1) (layer "F.Cu") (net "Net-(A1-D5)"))
 (segment (start 115.68 85.2) (end 99.481623 85.2) (width 1) (layer "F.Cu") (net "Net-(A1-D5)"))
 (segment (start 102.291623 76.99) (end 152.165433 76.99) (width 1) (layer "F.Cu") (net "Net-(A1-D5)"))
 (segment (start 118.38 82.5) (end 115.68 85.2) (width 1) (layer "F.Cu") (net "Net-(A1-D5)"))
 (segment (start 152.165433 76.99) (end 155.4 80.224567) (width 1) (layer "F.Cu") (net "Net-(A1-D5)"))
 (segment (start 99.1 83.121321) (end 99.1 81.878679) (width 1) (layer "F.Cu") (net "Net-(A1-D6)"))
 (segment (start 154.2 80.721623) (end 154.2 91.84) (width 1) (layer "F.Cu") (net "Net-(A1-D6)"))
 (segment (start 99.1 81.878679) (end 102.788679 78.19) (width 1) (layer "F.Cu") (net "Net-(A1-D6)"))
 (segment (start 154.2 91.84) (end 151.5 94.54) (width 1) (layer "F.Cu") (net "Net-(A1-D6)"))
 (segment (start 99.978679 84) (end 99.1 83.121321) (width 1) (layer "F.Cu") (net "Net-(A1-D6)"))
 (segment (start 151.668377 78.19) (end 154.2 80.721623) (width 1) (layer "F.Cu") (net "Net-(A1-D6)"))
 (segment (start 114.34 84) (end 99.978679 84) (width 1) (layer "F.Cu") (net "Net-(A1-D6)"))
 (segment (start 115.84 82.5) (end 114.34 84) (width 1) (layer "F.Cu") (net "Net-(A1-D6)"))
 (segment (start 102.788679 78.19) (end 151.668377 78.19) (width 1) (layer "F.Cu") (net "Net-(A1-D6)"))
 (segment (start 153 85.42) (end 151.5 86.92) (width 1) (layer "F.Cu") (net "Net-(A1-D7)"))
 (segment (start 153 81.218679) (end 153 85.42) (width 1) (layer "F.Cu") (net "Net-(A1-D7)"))
 (segment (start 151.171321 79.39) (end 153 81.218679) (width 1) (layer "F.Cu") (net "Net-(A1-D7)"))
 (segment (start 113.3 82.5) (end 116.41 79.39) (width 1) (layer "F.Cu") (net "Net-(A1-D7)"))
 (segment (start 116.41 79.39) (end 151.171321 79.39) (width 1) (layer "F.Cu") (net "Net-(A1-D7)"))
 (segment (start 148.8 79.14) (end 151.5 81.84) (width 1) (layer "B.Cu") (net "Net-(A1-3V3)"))
 (segment (start 103.14 97.74) (end 99.1 93.7) (width 1) (layer "B.Cu") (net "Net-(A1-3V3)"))
 (segment (start 99.1 81.878679) (end 101.838679 79.14) (width 1) (layer "B.Cu") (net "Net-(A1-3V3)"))
 (segment (start 153 83.34) (end 153 95.58) (width 1) (layer "B.Cu") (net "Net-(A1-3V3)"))
 (segment (start 153 95.58) (end 151.5 97.08) (width 1) (layer "B.Cu") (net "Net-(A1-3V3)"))
 (segment (start 101.838679 79.14) (end 148.8 79.14) (width 1) (layer "B.Cu") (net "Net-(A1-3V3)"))
 (segment (start 99.1 93.7) (end 99.1 81.878679) (width 1) (layer "B.Cu") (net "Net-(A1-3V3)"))
 (segment (start 151.5 81.84) (end 153 83.34) (width 1) (layer "B.Cu") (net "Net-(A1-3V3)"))
 (segment (start 142.19 103.69) (end 143.19 103.69) (width 0.75) (layer "F.Cu") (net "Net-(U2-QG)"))
 (segment (start 142 96.42) (end 142 103.5) (width 0.75) (layer "F.Cu") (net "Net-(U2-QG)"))
 (segment (start 143.88 94.54) (end 142 96.42) (width 0.75) (layer "F.Cu") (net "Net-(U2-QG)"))
 (segment (start 142 103.5) (end 142.19 103.69) (width 0.75) (layer "F.Cu") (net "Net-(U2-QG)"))
 (segment (start 144.265 112.385) (end 143.19 111.31) (width 0.75) (layer "F.Cu") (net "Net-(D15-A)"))
 (segment (start 144.265 116.25) (end 144.265 112.385) (width 0.75) (layer "F.Cu") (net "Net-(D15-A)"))
 (segment (start 143.88 86.92) (end 139.05 91.75) (width 0.75) (layer "F.Cu") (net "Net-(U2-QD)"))
 (segment (start 139.05 100.45) (end 138.5 101) (width 0.75) (layer "F.Cu") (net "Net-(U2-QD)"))
 (segment (start 121.19 101) (end 120.5 101.69) (width 0.75) (layer "F.Cu") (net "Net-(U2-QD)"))
 (segment (start 139.05 91.75) (end 139.05 100.45) (width 0.75) (layer "F.Cu") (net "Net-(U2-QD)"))
 (segment (start 120.5 101.69) (end 120.5 103.69) (width 0.75) (layer "F.Cu") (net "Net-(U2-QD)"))
 (segment (start 138.5 101) (end 121.19 101) (width 0.75) (layer "F.Cu") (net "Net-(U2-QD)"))
 (segment (start 97.615 101.115) (end 98.19 101.69) (width 0.75) (layer "F.Cu") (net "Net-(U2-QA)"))
 (segment (start 100.501953 94.55) (end 97.615 97.436953) (width 0.75) (layer "F.Cu") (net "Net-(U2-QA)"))
 (segment (start 151.5 84.38) (end 147.585 80.465) (width 0.75) (layer "F.Cu") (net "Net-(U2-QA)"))
 (segment (start 126.86 94.55) (end 100.501953 94.55) (width 0.75) (layer "F.Cu") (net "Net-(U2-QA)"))
 (segment (start 97.615 97.436953) (end 97.615 101.115) (width 0.75) (layer "F.Cu") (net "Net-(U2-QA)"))
 (segment (start 147.585 80.465) (end 140.945 80.465) (width 0.75) (layer "F.Cu") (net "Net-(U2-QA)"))
 (segment (start 98.19 101.69) (end 98.19 103.38) (width 0.75) (layer "F.Cu") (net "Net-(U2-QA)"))
 (segment (start 140.945 80.465) (end 126.86 94.55) (width 0.75) (layer "F.Cu") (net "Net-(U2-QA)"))
 (segment (start 98.19 103.38) (end 98.5 103.69) (width 0.75) (layer "F.Cu") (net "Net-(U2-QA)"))
 (segment (start 99.265 112.075) (end 98.5 111.31) (width 0.75) (layer "F.Cu") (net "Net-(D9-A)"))
 (segment (start 99.265 116.25) (end 99.265 112.075) (width 0.75) (layer "F.Cu") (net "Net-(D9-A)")))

